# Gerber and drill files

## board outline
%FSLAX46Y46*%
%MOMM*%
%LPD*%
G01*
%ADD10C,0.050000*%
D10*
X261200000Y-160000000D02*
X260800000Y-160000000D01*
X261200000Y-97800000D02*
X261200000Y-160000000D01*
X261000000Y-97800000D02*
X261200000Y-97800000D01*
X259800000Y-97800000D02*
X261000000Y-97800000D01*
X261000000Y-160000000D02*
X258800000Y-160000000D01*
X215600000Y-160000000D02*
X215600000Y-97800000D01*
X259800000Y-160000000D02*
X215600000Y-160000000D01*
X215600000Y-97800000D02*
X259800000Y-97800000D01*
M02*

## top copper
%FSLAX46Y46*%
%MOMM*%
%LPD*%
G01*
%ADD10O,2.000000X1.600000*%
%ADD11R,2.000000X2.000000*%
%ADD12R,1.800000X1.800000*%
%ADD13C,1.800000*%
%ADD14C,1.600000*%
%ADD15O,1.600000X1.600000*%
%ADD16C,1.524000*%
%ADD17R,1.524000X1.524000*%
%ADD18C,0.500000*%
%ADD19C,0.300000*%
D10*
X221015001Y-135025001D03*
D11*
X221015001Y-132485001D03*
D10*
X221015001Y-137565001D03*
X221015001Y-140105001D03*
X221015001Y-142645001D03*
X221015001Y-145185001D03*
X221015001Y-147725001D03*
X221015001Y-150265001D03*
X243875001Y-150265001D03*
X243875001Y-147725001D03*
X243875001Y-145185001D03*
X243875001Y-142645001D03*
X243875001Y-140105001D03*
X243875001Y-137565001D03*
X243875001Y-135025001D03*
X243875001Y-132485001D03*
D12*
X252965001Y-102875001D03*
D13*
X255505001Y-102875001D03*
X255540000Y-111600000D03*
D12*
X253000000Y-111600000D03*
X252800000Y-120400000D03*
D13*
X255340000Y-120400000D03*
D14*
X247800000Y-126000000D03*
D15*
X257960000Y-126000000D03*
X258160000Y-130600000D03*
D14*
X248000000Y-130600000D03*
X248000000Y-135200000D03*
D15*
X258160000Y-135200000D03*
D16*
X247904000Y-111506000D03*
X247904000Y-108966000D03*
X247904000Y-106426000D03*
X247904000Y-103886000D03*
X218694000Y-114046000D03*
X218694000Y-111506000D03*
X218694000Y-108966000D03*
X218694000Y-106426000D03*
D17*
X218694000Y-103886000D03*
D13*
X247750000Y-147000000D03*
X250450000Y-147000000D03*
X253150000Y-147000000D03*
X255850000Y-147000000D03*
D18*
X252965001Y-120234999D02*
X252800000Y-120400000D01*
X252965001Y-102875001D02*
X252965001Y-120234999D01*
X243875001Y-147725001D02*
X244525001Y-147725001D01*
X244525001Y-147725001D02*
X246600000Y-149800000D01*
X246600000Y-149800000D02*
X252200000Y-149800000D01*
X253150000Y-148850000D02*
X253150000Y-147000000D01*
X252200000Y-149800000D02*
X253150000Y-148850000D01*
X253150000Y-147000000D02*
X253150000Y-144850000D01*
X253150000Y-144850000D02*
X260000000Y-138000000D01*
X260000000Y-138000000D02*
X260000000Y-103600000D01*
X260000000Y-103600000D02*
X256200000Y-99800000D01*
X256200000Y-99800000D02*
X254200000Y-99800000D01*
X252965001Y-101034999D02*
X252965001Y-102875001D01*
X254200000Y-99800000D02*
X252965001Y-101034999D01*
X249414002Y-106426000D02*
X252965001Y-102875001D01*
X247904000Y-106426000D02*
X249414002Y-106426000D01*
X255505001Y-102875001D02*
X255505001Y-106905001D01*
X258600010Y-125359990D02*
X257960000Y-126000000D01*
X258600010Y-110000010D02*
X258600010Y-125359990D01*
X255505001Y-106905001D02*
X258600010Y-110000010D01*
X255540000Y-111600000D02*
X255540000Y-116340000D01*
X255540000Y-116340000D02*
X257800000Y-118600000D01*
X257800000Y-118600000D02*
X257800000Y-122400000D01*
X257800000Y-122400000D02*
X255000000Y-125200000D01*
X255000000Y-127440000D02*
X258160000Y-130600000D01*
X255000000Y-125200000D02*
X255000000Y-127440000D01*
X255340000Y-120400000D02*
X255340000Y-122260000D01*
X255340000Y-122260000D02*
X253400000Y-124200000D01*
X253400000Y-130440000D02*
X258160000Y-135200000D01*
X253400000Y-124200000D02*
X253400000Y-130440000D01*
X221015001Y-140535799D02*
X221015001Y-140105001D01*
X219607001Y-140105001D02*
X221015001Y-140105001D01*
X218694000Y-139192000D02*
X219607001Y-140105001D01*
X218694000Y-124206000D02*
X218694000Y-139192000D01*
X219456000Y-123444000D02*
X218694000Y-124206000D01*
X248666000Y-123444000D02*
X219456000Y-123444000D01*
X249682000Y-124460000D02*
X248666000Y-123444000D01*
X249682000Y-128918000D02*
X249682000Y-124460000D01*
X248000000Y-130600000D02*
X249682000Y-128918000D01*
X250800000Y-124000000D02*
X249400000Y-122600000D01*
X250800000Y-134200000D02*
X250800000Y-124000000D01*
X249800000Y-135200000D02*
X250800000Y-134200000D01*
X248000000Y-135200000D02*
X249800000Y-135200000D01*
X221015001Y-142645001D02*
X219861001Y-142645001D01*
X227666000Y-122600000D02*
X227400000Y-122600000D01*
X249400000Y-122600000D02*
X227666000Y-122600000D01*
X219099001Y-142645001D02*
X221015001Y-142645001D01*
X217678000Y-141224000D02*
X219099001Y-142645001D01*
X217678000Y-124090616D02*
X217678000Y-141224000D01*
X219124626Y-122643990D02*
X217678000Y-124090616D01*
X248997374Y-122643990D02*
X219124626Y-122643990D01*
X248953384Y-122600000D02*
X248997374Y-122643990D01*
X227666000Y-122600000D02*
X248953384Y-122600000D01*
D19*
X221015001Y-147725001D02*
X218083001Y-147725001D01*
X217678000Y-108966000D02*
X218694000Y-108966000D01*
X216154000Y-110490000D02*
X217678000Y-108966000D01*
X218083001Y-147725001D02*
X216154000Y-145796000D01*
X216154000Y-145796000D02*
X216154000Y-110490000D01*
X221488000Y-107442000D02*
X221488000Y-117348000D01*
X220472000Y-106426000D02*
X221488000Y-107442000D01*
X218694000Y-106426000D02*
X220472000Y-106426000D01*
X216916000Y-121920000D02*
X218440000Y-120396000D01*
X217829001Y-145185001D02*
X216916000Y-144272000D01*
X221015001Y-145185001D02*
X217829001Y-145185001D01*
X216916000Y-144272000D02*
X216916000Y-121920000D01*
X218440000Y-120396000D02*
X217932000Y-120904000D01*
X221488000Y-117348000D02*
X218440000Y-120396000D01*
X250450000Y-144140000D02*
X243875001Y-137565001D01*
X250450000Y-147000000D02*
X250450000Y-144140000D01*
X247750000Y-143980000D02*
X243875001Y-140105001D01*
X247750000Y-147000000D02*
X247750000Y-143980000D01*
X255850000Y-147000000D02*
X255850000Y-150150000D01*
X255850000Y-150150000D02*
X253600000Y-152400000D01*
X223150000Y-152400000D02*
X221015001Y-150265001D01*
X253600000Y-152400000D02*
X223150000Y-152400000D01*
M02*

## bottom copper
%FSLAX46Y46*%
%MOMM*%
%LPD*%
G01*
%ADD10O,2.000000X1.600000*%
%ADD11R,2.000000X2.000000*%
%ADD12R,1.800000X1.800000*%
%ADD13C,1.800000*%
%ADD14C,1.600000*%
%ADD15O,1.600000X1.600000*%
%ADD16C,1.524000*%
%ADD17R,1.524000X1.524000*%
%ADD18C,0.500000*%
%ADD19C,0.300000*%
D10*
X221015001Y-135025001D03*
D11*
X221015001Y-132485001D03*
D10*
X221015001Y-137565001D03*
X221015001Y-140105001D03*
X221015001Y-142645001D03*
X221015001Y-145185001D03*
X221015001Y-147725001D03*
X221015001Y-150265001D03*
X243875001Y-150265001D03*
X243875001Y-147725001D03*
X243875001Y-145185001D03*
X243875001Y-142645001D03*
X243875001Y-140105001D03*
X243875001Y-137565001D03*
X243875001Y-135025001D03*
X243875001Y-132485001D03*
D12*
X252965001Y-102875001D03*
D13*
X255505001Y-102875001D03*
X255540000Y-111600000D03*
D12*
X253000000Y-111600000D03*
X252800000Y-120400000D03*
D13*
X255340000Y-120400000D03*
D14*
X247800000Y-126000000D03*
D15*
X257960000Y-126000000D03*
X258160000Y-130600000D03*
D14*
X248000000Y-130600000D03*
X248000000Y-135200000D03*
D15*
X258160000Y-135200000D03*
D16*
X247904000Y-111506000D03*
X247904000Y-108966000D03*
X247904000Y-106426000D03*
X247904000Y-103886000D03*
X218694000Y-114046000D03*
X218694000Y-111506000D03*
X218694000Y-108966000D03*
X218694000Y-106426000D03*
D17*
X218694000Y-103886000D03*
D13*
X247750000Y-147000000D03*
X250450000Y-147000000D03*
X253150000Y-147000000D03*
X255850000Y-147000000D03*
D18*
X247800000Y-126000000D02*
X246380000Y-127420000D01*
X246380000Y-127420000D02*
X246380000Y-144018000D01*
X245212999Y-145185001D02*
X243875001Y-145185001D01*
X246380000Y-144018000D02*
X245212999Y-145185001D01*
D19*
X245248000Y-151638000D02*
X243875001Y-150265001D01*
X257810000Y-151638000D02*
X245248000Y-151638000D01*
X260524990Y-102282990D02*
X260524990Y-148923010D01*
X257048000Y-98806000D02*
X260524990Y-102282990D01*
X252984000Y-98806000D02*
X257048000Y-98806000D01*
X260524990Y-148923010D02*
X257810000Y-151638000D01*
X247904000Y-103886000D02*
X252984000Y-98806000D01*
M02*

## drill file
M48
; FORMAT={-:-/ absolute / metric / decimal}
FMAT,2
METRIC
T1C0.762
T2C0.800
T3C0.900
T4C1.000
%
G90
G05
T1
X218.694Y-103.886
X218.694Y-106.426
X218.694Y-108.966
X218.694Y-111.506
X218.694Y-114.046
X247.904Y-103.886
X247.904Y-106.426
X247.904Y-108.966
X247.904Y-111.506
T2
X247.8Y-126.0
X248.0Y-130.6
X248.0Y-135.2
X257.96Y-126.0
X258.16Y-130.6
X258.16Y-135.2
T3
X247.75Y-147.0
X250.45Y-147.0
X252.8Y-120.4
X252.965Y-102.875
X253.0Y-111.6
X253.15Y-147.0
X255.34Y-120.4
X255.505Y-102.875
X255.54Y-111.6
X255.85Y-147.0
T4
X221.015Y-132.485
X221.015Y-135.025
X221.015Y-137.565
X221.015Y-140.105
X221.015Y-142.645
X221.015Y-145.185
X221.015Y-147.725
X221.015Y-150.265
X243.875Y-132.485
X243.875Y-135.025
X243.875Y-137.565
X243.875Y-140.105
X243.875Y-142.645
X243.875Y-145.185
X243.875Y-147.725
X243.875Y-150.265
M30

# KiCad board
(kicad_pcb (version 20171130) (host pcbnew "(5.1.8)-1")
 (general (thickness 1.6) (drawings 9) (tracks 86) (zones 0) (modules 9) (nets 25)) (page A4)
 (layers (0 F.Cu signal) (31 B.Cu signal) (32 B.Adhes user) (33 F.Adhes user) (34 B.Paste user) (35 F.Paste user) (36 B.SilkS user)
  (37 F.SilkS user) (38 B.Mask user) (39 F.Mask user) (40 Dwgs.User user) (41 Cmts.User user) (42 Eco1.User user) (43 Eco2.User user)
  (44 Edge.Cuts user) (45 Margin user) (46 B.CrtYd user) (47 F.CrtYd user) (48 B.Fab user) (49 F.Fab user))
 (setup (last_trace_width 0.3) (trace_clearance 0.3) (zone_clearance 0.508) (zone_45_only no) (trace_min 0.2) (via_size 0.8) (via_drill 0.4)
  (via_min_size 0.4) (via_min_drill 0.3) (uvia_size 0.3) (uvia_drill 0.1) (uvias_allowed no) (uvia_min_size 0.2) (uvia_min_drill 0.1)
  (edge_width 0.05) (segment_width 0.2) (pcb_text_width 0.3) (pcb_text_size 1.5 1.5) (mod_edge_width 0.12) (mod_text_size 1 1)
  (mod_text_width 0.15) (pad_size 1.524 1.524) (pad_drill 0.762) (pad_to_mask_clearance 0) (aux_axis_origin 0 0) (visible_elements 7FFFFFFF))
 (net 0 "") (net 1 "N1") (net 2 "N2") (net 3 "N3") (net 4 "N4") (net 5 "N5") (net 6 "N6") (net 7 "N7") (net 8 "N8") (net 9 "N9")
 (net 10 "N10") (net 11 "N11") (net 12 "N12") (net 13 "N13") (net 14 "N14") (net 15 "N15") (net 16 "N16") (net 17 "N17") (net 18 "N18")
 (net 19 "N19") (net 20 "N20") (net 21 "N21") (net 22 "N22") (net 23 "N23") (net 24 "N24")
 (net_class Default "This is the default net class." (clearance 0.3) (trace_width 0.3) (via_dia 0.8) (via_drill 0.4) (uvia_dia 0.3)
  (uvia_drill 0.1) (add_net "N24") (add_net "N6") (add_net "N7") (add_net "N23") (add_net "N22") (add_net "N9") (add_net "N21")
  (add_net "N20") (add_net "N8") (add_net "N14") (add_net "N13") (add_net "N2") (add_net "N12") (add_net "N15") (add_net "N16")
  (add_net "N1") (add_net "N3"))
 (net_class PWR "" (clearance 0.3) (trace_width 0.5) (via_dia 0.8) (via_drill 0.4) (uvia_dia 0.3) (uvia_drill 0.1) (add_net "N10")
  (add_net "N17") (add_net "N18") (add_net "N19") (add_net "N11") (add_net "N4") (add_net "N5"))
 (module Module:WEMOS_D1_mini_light (layer F.Cu) (at 221.015001 132.485001)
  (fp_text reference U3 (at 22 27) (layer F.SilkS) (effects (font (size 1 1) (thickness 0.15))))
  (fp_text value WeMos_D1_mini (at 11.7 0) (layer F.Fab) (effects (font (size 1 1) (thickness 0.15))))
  (pad 2 thru_hole oval (at 0 2.54) (size 2 1.6) (drill 1) (layers *.Cu *.Mask) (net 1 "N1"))
  (pad 1 thru_hole rect (at 0 0) (size 2 2) (drill 1) (layers *.Cu *.Mask) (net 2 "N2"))
  (pad 3 thru_hole oval (at 0 5.08) (size 2 1.6) (drill 1) (layers *.Cu *.Mask) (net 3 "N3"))
  (pad 4 thru_hole oval (at 0 7.62) (size 2 1.6) (drill 1) (layers *.Cu *.Mask) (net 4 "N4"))
  (pad 5 thru_hole oval (at 0 10.16) (size 2 1.6) (drill 1) (layers *.Cu *.Mask) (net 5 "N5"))
  (pad 6 thru_hole oval (at 0 12.7) (size 2 1.6) (drill 1) (layers *.Cu *.Mask) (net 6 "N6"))
  (pad 7 thru_hole oval (at 0 15.24) (size 2 1.6) (drill 1) (layers *.Cu *.Mask) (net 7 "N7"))
  (pad 8 thru_hole oval (at 0 17.78) (size 2 1.6) (drill 1) (layers *.Cu *.Mask) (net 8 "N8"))
  (pad 9 thru_hole oval (at 22.86 17.78) (size 2 1.6) (drill 1) (layers *.Cu *.Mask) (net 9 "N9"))
  (pad 10 thru_hole oval (at 22.86 15.24) (size 2 1.6) (drill 1) (layers *.Cu *.Mask) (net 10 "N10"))
  (pad 11 thru_hole oval (at 22.86 12.7) (size 2 1.6) (drill 1) (layers *.Cu *.Mask) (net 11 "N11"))
  (pad 12 thru_hole oval (at 22.86 10.16) (size 2 1.6) (drill 1) (layers *.Cu *.Mask) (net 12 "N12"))
  (pad 13 thru_hole oval (at 22.86 7.62) (size 2 1.6) (drill 1) (layers *.Cu *.Mask) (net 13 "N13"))
  (pad 14 thru_hole oval (at 22.86 5.08) (size 2 1.6) (drill 1) (layers *.Cu *.Mask) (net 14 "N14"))
  (pad 15 thru_hole oval (at 22.86 2.54) (size 2 1.6) (drill 1) (layers *.Cu *.Mask) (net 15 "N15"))
  (pad 16 thru_hole oval (at 22.86 0) (size 2 1.6) (drill 1) (layers *.Cu *.Mask) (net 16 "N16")))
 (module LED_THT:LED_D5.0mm (layer F.Cu) (at 252.965001 102.875001)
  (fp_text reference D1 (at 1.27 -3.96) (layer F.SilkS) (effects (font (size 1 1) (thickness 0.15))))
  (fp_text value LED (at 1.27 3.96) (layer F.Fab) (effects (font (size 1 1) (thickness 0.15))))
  (pad 1 thru_hole rect (at 0 0) (size 1.8 1.8) (drill 0.9) (layers *.Cu *.Mask) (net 10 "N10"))
  (pad 2 thru_hole circle (at 2.54 0) (size 1.8 1.8) (drill 0.9) (layers *.Cu *.Mask) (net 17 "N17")))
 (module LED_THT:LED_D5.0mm (layer F.Cu) (at 253 111.6)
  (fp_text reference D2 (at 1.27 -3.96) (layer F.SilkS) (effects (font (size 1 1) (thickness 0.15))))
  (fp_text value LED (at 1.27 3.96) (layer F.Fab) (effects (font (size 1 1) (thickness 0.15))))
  (pad 2 thru_hole circle (at 2.54 0) (size 1.8 1.8) (drill 0.9) (layers *.Cu *.Mask) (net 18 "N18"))
  (pad 1 thru_hole rect (at 0 0) (size 1.8 1.8) (drill 0.9) (layers *.Cu *.Mask) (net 10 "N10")))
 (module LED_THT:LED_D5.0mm (layer F.Cu) (at 252.8 120.4)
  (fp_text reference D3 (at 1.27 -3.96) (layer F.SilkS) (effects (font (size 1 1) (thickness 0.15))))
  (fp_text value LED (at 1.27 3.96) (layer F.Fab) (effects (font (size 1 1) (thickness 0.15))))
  (pad 1 thru_hole rect (at 0 0) (size 1.8 1.8) (drill 0.9) (layers *.Cu *.Mask) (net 10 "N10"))
  (pad 2 thru_hole circle (at 2.54 0) (size 1.8 1.8) (drill 0.9) (layers *.Cu *.Mask) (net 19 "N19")))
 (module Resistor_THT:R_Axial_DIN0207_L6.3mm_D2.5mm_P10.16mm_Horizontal (layer F.Cu) (at 247.8 126)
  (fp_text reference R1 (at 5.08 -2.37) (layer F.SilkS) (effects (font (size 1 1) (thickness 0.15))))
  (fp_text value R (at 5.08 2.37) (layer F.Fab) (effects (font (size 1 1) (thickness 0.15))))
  (pad 1 thru_hole circle (at 0 0) (size 1.6 1.6) (drill 0.8) (layers *.Cu *.Mask) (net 11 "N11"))
  (pad 2 thru_hole oval (at 10.16 0) (size 1.6 1.6) (drill 0.8) (layers *.Cu *.Mask) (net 17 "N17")))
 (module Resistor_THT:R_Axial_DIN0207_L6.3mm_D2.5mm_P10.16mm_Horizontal (layer F.Cu) (at 248 130.6)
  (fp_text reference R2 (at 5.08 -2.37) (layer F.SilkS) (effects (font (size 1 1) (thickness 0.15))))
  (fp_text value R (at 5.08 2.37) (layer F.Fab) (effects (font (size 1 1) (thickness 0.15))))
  (pad 2 thru_hole oval (at 10.16 0) (size 1.6 1.6) (drill 0.8) (layers *.Cu *.Mask) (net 18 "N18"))
  (pad 1 thru_hole circle (at 0 0) (size 1.6 1.6) (drill 0.8) (layers *.Cu *.Mask) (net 4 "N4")))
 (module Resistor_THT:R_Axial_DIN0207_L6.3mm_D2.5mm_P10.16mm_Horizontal (layer F.Cu) (at 248 135.2)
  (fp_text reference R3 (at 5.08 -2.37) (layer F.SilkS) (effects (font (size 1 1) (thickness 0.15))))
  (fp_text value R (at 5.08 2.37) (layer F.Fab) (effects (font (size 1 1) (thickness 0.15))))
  (pad 1 thru_hole circle (at 0 0) (size 1.6 1.6) (drill 0.8) (layers *.Cu *.Mask) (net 5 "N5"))
  (pad 2 thru_hole oval (at 10.16 0) (size 1.6 1.6) (drill 0.8) (layers *.Cu *.Mask) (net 19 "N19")))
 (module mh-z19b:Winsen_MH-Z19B (layer F.Cu) (at 218.694 117.856 180)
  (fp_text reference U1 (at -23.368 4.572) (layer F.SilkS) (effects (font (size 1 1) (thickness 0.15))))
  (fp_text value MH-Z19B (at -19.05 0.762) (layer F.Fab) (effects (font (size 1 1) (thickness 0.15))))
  (pad 9 thru_hole circle (at -29.21 6.35 180) (size 1.524 1.524) (drill 0.762) (layers *.Cu *.Mask) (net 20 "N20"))
  (pad 8 thru_hole circle (at -29.21 8.89 180) (size 1.524 1.524) (drill 0.762) (layers *.Cu *.Mask) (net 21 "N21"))
  (pad 7 thru_hole circle (at -29.21 11.43 180) (size 1.524 1.524) (drill 0.762) (layers *.Cu *.Mask) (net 10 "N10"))
  (pad 6 thru_hole circle (at -29.21 13.97 180) (size 1.524 1.524) (drill 0.762) (layers *.Cu *.Mask) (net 9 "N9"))
  (pad 5 thru_hole circle (at 0 3.81 180) (size 1.524 1.524) (drill 0.762) (layers *.Cu *.Mask) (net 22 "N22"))
  (pad 4 thru_hole circle (at 0 6.35 180) (size 1.524 1.524) (drill 0.762) (layers *.Cu *.Mask) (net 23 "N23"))
  (pad 3 thru_hole circle (at 0 8.89 180) (size 1.524 1.524) (drill 0.762) (layers *.Cu *.Mask) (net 7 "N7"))
  (pad 2 thru_hole circle (at 0 11.43 180) (size 1.524 1.524) (drill 0.762) (layers *.Cu *.Mask) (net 6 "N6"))
  (pad 1 thru_hole rect (at 0 13.97 180) (size 1.524 1.524) (drill 0.762) (layers *.Cu *.Mask) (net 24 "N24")))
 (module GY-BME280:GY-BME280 (layer F.Cu) (at 251.8 149 180)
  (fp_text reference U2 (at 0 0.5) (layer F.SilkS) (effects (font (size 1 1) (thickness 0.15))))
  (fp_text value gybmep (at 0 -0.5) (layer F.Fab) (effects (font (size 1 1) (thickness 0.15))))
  (pad 4 thru_hole circle (at 4.05 2 180) (size 1.8 1.8) (drill 0.9) (layers *.Cu *.Mask) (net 13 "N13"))
  (pad 3 thru_hole circle (at 1.35 2 180) (size 1.8 1.8) (drill 0.9) (layers *.Cu *.Mask) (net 14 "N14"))
  (pad 2 thru_hole circle (at -1.35 2 180) (size 1.8 1.8) (drill 0.9) (layers *.Cu *.Mask) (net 10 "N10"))
  (pad 1 thru_hole circle (at -4.05 2 180) (size 1.8 1.8) (drill 0.9) (layers *.Cu *.Mask) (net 8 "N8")))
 (gr_line (start 261.2 160) (end 260.8 160) (layer Edge.Cuts) (width 0.05))
 (gr_line (start 261.2 97.8) (end 261.2 160) (layer Edge.Cuts) (width 0.05))
 (gr_line (start 261 97.8) (end 261.2 97.8) (layer Edge.Cuts) (width 0.05))
 (gr_line (start 259.8 97.8) (end 261 97.8) (layer Edge.Cuts) (width 0.05))
 (gr_line (start 261 160) (end 258.8 160) (layer Edge.Cuts) (width 0.05))
 (gr_line (start 215.6 160) (end 215.6 97.8) (layer Edge.Cuts) (width 0.05))
 (gr_line (start 259.8 160) (end 215.6 160) (layer Edge.Cuts) (width 0.05))
 (gr_line (start 215.6 97.8) (end 259.8 97.8) (layer Edge.Cuts) (width 0.05))
 (segment (start 252.965001 120.234999) (end 252.8 120.4) (width 0.5) (layer F.Cu) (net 10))
 (segment (start 252.965001 102.875001) (end 252.965001 120.234999) (width 0.5) (layer F.Cu) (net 10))
 (segment (start 243.875001 147.725001) (end 244.525001 147.725001) (width 0.5) (layer F.Cu) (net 10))
 (segment (start 244.525001 147.725001) (end 246.6 149.8) (width 0.5) (layer F.Cu) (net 10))
 (segment (start 246.6 149.8) (end 252.2 149.8) (width 0.5) (layer F.Cu) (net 10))
 (segment (start 253.15 148.85) (end 253.15 147) (width 0.5) (layer F.Cu) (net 10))
 (segment (start 252.2 149.8) (end 253.15 148.85) (width 0.5) (layer F.Cu) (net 10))
 (segment (start 253.15 147) (end 253.15 144.85) (width 0.5) (layer F.Cu) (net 10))
 (segment (start 253.15 144.85) (end 260 138) (width 0.5) (layer F.Cu) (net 10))
 (segment (start 260 138) (end 260 103.6) (width 0.5) (layer F.Cu) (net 10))
 (segment (start 260 103.6) (end 256.2 99.8) (width 0.5) (layer F.Cu) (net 10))
 (segment (start 256.2 99.8) (end 254.2 99.8) (width 0.5) (layer F.Cu) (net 10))
 (segment (start 252.965001 101.034999) (end 252.965001 102.875001) (width 0.5) (layer F.Cu) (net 10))
 (segment (start 254.2 99.8) (end 252.965001 101.034999) (width 0.5) (layer F.Cu) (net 10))
 (segment (start 249.414002 106.426) (end 252.965001 102.875001) (width 0.5) (layer F.Cu) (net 10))
 (segment (start 247.904 106.426) (end 249.414002 106.426) (width 0.5) (layer F.Cu) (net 10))
 (segment (start 255.505001 102.875001) (end 255.505001 106.905001) (width 0.5) (layer F.Cu) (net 17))
 (segment (start 258.60001 125.35999) (end 257.96 126) (width 0.5) (layer F.Cu) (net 17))
 (segment (start 258.60001 110.00001) (end 258.60001 125.35999) (width 0.5) (layer F.Cu) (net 17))
 (segment (start 255.505001 106.905001) (end 258.60001 110.00001) (width 0.5) (layer F.Cu) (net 17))
 (segment (start 255.54 111.6) (end 255.54 116.34) (width 0.5) (layer F.Cu) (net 18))
 (segment (start 255.54 116.34) (end 257.8 118.6) (width 0.5) (layer F.Cu) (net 18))
 (segment (start 257.8 118.6) (end 257.8 122.4) (width 0.5) (layer F.Cu) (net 18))
 (segment (start 257.8 122.4) (end 255 125.2) (width 0.5) (layer F.Cu) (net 18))
 (segment (start 255 127.44) (end 258.16 130.6) (width 0.5) (layer F.Cu) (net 18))
 (segment (start 255 125.2) (end 255 127.44) (width 0.5) (layer F.Cu) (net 18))
 (segment (start 255.34 120.4) (end 255.34 122.26) (width 0.5) (layer F.Cu) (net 19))
 (segment (start 255.34 122.26) (end 253.4 124.2) (width 0.5) (layer F.Cu) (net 19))
 (segment (start 253.4 130.44) (end 258.16 135.2) (width 0.5) (layer F.Cu) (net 19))
 (segment (start 253.4 124.2) (end 253.4 130.44) (width 0.5) (layer F.Cu) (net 19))
 (segment (start 247.8 126) (end 246.38 127.42) (width 0.5) (layer B.Cu) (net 11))
 (segment (start 246.38 127.42) (end 246.38 144.018) (width 0.5) (layer B.Cu) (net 11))
 (segment (start 245.212999 145.185001) (end 243.875001 145.185001) (width 0.5) (layer B.Cu) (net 11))
 (segment (start 246.38 144.018) (end 245.212999 145.185001) (width 0.5) (layer B.Cu) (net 11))
 (segment (start 221.015001 140.535799) (end 221.015001 140.105001) (width 0.5) (layer F.Cu) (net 4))
 (segment (start 219.607001 140.105001) (end 221.015001 140.105001) (width 0.5) (layer F.Cu) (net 4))
 (segment (start 218.694 139.192) (end 219.607001 140.105001) (width 0.5) (layer F.Cu) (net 4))
 (segment (start 218.694 124.206) (end 218.694 139.192) (width 0.5) (layer F.Cu) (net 4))
 (segment (start 219.456 123.444) (end 218.694 124.206) (width 0.5) (layer F.Cu) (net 4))
 (segment (start 248.666 123.444) (end 219.456 123.444) (width 0.5) (layer F.Cu) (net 4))
 (segment (start 249.682 124.46) (end 248.666 123.444) (width 0.5) (layer F.Cu) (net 4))
 (segment (start 249.682 128.918) (end 249.682 124.46) (width 0.5) (layer F.Cu) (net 4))
 (segment (start 248 130.6) (end 249.682 128.918) (width 0.5) (layer F.Cu) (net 4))
 (segment (start 250.8 124) (end 249.4 122.6) (width 0.5) (layer F.Cu) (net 5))
 (segment (start 250.8 134.2) (end 250.8 124) (width 0.5) (layer F.Cu) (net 5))
 (segment (start 249.8 135.2) (end 250.8 134.2) (width 0.5) (layer F.Cu) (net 5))
 (segment (start 248 135.2) (end 249.8 135.2) (width 0.5) (layer F.Cu) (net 5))
 (segment (start 221.015001 142.645001) (end 219.861001 142.645001) (width 0.5) (layer F.Cu) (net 5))
 (segment (start 227.666 122.6) (end 227.4 122.6) (width 0.5) (layer F.Cu) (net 5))
 (segment (start 249.4 122.6) (end 227.666 122.6) (width 0.5) (layer F.Cu) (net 5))
 (segment (start 219.099001 142.645001) (end 221.015001 142.645001) (width 0.5) (layer F.Cu) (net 5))
 (segment (start 217.678 141.224) (end 219.099001 142.645001) (width 0.5) (layer F.Cu) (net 5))
 (segment (start 217.678 124.090616) (end 217.678 141.224) (width 0.5) (layer F.Cu) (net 5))
 (segment (start 219.124626 122.64399) (end 217.678 124.090616) (width 0.5) (layer F.Cu) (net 5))
 (segment (start 248.997374 122.64399) (end 219.124626 122.64399) (width 0.5) (layer F.Cu) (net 5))
 (segment (start 248.953384 122.6) (end 248.997374 122.64399) (width 0.5) (layer F.Cu) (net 5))
 (segment (start 227.666 122.6) (end 248.953384 122.6) (width 0.5) (layer F.Cu) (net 5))
 (segment (start 245.248 151.638) (end 243.875001 150.265001) (width 0.3) (layer B.Cu) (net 9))
 (segment (start 257.81 151.638) (end 245.248 151.638) (width 0.3) (layer B.Cu) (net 9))
 (segment (start 260.52499 102.28299) (end 260.52499 148.92301) (width 0.3) (layer B.Cu) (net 9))
 (segment (start 257.048 98.806) (end 260.52499 102.28299) (width 0.3) (layer B.Cu) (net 9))
 (segment (start 252.984 98.806) (end 257.048 98.806) (width 0.3) (layer B.Cu) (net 9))
 (segment (start 260.52499 148.92301) (end 257.81 151.638) (width 0.3) (layer B.Cu) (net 9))
 (segment (start 247.904 103.886) (end 252.984 98.806) (width 0.3) (layer B.Cu) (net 9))
 (segment (start 221.015001 147.725001) (end 218.083001 147.725001) (width 0.3) (layer F.Cu) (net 7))
 (segment (start 217.678 108.966) (end 218.694 108.966) (width 0.3) (layer F.Cu) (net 7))
 (segment (start 216.154 110.49) (end 217.678 108.966) (width 0.3) (layer F.Cu) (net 7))
 (segment (start 218.083001 147.725001) (end 216.154 145.796) (width 0.3) (layer F.Cu) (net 7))
 (segment (start 216.154 145.796) (end 216.154 110.49) (width 0.3) (layer F.Cu) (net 7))
 (segment (start 221.488 107.442) (end 221.488 117.348) (width 0.3) (layer F.Cu) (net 6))
 (segment (start 220.472 106.426) (end 221.488 107.442) (width 0.3) (layer F.Cu) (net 6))
 (segment (start 218.694 106.426) (end 220.472 106.426) (width 0.3) (layer F.Cu) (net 6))
 (segment (start 216.916 121.92) (end 218.44 120.396) (width 0.3) (layer F.Cu) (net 6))
 (segment (start 217.829001 145.185001) (end 216.916 144.272) (width 0.3) (layer F.Cu) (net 6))
 (segment (start 221.015001 145.185001) (end 217.829001 145.185001) (width 0.3) (layer F.Cu) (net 6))
 (segment (start 216.916 144.272) (end 216.916 121.92) (width 0.3) (layer F.Cu) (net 6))
 (segment (start 218.44 120.396) (end 217.932 120.904) (width 0.3) (layer F.Cu) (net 6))
 (segment (start 221.488 117.348) (end 218.44 120.396) (width 0.3) (layer F.Cu) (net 6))
 (segment (start 250.45 144.14) (end 243.875001 137.565001) (width 0.3) (layer F.Cu) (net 14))
 (segment (start 250.45 147) (end 250.45 144.14) (width 0.3) (layer F.Cu) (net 14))
 (segment (start 247.75 143.98) (end 243.875001 140.105001) (width 0.3) (layer F.Cu) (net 13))
 (segment (start 247.75 147) (end 247.75 143.98) (width 0.3) (layer F.Cu) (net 13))
 (segment (start 255.85 147) (end 255.85 150.15) (width 0.3) (layer F.Cu) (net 8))
 (segment (start 255.85 150.15) (end 253.6 152.4) (width 0.3) (layer F.Cu) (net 8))
 (segment (start 223.15 152.4) (end 221.015001 150.265001) (width 0.3) (layer F.Cu) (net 8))
 (segment (start 253.6 152.4) (end 223.15 152.4) (width 0.3) (layer F.Cu) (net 8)))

